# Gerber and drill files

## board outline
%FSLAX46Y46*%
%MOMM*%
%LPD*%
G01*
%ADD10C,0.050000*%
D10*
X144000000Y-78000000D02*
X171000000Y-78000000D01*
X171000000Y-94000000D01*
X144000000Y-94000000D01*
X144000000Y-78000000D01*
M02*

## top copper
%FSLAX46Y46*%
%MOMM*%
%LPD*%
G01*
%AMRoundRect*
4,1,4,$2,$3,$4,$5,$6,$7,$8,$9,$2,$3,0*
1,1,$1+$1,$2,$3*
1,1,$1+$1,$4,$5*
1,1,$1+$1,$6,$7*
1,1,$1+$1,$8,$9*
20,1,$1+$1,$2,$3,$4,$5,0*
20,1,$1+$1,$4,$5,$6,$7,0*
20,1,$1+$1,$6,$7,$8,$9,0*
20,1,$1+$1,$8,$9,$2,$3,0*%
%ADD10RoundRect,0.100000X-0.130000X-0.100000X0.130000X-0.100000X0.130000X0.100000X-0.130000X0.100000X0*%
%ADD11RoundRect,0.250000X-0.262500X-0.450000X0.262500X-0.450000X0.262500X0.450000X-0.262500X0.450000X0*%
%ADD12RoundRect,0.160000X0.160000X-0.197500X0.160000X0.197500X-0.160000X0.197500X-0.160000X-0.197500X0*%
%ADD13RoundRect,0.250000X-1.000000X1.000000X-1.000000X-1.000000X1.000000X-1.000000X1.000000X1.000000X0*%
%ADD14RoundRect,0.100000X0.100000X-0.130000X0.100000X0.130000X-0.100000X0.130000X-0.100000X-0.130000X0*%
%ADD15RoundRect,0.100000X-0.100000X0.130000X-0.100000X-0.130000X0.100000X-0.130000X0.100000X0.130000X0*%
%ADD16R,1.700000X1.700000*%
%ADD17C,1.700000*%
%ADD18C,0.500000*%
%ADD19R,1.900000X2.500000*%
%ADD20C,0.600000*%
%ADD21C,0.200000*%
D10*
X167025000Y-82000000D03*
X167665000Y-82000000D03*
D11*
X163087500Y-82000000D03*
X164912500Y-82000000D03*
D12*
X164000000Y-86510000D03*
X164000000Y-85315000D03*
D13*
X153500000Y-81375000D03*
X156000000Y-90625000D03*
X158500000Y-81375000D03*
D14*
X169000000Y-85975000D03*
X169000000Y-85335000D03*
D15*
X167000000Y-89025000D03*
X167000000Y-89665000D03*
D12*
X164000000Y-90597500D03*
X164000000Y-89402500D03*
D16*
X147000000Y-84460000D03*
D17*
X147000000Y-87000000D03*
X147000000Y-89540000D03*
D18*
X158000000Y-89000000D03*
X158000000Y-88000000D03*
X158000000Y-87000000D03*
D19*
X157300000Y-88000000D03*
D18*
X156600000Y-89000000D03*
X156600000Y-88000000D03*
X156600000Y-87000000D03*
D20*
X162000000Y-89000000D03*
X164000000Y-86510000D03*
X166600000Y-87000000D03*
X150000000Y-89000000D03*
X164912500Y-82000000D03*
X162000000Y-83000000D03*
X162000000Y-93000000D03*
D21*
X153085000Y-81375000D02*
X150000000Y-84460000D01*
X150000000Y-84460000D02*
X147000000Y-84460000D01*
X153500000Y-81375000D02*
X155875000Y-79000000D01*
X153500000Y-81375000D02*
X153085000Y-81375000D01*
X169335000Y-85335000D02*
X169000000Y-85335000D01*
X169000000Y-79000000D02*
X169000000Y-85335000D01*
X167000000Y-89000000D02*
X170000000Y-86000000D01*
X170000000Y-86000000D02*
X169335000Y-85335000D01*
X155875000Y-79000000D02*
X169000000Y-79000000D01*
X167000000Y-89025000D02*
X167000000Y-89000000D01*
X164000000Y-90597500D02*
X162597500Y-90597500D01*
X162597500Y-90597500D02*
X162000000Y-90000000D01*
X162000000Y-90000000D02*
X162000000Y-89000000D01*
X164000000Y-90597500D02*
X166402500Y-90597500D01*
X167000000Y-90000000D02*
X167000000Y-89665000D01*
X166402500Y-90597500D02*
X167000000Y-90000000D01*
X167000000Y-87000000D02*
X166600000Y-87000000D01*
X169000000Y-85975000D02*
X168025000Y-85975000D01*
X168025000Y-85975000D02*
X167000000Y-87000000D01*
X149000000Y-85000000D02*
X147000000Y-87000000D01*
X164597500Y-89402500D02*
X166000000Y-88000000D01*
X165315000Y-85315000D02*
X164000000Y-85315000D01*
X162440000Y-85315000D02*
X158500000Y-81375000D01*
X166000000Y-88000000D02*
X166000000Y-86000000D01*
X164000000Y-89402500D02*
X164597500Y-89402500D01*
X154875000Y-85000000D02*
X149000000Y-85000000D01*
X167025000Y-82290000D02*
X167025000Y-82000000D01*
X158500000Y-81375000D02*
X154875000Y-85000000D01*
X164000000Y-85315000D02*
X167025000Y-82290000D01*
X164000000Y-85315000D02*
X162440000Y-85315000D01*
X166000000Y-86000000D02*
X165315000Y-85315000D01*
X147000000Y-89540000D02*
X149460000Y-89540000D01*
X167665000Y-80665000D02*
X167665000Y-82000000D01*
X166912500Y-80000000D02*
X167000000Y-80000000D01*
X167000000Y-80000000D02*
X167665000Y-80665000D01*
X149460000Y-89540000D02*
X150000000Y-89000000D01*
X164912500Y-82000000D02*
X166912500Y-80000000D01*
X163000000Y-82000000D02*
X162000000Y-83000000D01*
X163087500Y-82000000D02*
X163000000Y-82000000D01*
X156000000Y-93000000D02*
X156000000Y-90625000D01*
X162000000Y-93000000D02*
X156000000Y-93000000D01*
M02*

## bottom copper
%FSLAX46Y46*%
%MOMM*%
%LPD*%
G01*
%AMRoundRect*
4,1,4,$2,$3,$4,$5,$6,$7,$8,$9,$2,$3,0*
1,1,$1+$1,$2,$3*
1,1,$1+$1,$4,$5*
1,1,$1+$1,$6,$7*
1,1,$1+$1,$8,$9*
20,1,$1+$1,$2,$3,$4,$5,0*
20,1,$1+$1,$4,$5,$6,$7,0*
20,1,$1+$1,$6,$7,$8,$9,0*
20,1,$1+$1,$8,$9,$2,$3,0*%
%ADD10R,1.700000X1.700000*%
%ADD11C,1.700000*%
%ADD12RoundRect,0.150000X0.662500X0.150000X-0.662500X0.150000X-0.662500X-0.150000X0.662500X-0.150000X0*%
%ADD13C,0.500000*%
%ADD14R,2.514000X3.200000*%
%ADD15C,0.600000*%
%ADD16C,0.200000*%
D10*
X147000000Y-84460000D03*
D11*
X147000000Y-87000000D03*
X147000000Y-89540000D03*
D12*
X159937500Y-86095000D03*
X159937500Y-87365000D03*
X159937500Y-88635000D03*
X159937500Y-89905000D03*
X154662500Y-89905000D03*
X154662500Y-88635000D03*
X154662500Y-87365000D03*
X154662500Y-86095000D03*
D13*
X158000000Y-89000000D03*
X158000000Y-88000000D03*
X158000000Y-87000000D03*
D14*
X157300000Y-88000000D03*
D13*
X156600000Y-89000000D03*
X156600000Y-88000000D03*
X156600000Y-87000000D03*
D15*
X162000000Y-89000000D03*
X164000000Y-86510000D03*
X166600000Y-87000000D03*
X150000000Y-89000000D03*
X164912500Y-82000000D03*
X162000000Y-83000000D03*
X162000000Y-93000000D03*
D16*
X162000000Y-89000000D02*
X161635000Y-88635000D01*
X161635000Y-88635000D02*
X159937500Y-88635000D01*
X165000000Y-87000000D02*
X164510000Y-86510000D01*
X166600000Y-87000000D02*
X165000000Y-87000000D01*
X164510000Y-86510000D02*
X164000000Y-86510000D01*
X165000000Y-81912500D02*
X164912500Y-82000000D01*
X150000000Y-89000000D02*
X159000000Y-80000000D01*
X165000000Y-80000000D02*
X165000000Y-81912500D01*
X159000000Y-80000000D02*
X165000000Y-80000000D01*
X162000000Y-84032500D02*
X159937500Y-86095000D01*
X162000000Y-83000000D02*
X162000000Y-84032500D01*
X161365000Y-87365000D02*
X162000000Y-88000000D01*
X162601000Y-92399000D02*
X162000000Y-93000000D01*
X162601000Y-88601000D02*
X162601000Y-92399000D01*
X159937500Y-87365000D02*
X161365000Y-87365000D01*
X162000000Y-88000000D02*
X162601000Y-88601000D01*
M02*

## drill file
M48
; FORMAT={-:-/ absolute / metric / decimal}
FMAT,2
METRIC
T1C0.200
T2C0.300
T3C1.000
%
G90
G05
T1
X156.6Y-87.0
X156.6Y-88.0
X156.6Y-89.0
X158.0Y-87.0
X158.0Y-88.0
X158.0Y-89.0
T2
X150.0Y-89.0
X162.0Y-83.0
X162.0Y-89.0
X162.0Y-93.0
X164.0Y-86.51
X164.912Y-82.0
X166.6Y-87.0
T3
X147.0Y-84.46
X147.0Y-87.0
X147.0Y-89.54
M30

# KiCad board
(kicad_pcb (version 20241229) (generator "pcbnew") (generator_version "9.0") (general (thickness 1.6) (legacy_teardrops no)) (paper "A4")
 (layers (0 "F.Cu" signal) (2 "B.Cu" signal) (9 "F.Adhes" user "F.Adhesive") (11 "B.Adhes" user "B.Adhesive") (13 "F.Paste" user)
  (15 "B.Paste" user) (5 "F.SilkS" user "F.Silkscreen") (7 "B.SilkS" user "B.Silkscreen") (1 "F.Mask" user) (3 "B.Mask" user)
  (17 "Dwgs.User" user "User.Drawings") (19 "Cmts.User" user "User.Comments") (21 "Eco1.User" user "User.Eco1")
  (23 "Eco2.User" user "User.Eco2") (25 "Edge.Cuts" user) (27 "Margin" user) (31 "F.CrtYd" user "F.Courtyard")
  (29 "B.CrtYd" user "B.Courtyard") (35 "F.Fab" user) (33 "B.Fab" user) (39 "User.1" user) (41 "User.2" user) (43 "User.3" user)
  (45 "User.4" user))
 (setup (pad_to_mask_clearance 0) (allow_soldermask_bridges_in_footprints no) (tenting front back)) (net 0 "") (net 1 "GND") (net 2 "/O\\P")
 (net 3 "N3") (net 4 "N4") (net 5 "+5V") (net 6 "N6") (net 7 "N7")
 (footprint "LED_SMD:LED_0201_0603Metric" (layer "F.Cu") (at 167.345 82)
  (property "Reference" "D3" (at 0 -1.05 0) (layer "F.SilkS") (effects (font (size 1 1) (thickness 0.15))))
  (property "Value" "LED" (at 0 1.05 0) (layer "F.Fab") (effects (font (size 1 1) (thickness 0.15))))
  (pad "" smd roundrect (at -0.345 0) (size 0.318 0.36) (layers "F.Paste") (roundrect_rratio 0.25))
  (pad "" smd roundrect (at 0.345 0) (size 0.318 0.36) (layers "F.Paste") (roundrect_rratio 0.25))
  (pad "1" smd roundrect (at -0.32 0) (size 0.46 0.4) (layers "F.Cu" "F.Mask") (roundrect_rratio 0.25) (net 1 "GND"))
  (pad "2" smd roundrect (at 0.32 0) (size 0.46 0.4) (layers "F.Cu" "F.Mask") (roundrect_rratio 0.25) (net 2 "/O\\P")))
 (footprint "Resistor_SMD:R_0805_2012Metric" (layer "F.Cu") (at 164 82)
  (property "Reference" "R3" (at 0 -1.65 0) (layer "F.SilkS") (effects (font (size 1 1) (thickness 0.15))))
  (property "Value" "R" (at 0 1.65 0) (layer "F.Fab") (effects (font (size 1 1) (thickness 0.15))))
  (pad "1" smd roundrect (at -0.9125 0) (size 1.025 1.4) (layers "F.Cu" "F.Mask" "F.Paste") (roundrect_rratio 0.243902) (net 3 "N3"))
  (pad "2" smd roundrect (at 0.9125 0) (size 1.025 1.4) (layers "F.Cu" "F.Mask" "F.Paste") (roundrect_rratio 0.243902) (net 2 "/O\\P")))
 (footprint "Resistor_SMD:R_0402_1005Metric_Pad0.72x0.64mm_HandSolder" (layer "F.Cu") (at 164 85.9125 90)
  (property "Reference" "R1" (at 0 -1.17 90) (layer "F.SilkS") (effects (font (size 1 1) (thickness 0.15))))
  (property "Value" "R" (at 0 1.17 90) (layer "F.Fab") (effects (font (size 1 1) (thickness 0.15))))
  (pad "1" smd roundrect (at -0.5975 0 90) (size 0.715 0.64) (layers "F.Cu" "F.Mask" "F.Paste") (roundrect_rratio 0.25) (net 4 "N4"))
  (pad "2" smd roundrect (at 0.5975 0 90) (size 0.715 0.64) (layers "F.Cu" "F.Mask" "F.Paste") (roundrect_rratio 0.25) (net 1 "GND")))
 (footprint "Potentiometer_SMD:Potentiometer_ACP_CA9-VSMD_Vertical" (layer "F.Cu") (at 156 86 -90)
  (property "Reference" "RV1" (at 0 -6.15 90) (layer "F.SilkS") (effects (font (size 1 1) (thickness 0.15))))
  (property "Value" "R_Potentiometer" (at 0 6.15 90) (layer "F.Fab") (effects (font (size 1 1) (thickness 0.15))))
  (pad "1" smd roundrect (at -4.625 2.5 270) (size 2.5 2.5) (layers "F.Cu" "F.Mask" "F.Paste") (roundrect_rratio 0.1) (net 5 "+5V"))
  (pad "2" smd roundrect (at 4.625 0 270) (size 2.5 2.5) (layers "F.Cu" "F.Mask" "F.Paste") (roundrect_rratio 0.1) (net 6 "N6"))
  (pad "3" smd roundrect (at -4.625 -2.5 270) (size 2.5 2.5) (layers "F.Cu" "F.Mask" "F.Paste") (roundrect_rratio 0.1) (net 1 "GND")))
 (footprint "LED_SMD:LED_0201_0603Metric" (layer "F.Cu") (at 169 85.655 90)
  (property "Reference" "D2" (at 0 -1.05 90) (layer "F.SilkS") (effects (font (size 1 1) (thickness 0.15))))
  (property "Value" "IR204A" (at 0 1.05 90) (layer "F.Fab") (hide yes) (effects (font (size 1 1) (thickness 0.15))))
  (pad "" smd roundrect (at -0.345 0 90) (size 0.318 0.36) (layers "F.Paste") (roundrect_rratio 0.25))
  (pad "" smd roundrect (at 0.345 0 90) (size 0.318 0.36) (layers "F.Paste") (roundrect_rratio 0.25))
  (pad "1" smd roundrect (at -0.32 0 90) (size 0.46 0.4) (layers "F.Cu" "F.Mask") (roundrect_rratio 0.25) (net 4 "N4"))
  (pad "2" smd roundrect (at 0.32 0 90) (size 0.46 0.4) (layers "F.Cu" "F.Mask") (roundrect_rratio 0.25) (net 5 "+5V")))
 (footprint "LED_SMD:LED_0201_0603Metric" (layer "F.Cu") (at 167 89.345 -90)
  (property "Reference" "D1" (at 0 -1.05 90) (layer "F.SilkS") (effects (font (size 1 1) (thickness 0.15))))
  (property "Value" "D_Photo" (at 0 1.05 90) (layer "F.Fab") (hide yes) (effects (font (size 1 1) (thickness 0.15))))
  (pad "" smd roundrect (at -0.345 0 270) (size 0.318 0.36) (layers "F.Paste") (roundrect_rratio 0.25))
  (pad "" smd roundrect (at 0.345 0 270) (size 0.318 0.36) (layers "F.Paste") (roundrect_rratio 0.25))
  (pad "1" smd roundrect (at -0.32 0 270) (size 0.46 0.4) (layers "F.Cu" "F.Mask") (roundrect_rratio 0.25) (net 5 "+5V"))
  (pad "2" smd roundrect (at 0.32 0 270) (size 0.46 0.4) (layers "F.Cu" "F.Mask") (roundrect_rratio 0.25) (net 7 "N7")))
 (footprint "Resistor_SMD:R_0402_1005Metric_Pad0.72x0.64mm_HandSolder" (layer "F.Cu") (at 164 90 90)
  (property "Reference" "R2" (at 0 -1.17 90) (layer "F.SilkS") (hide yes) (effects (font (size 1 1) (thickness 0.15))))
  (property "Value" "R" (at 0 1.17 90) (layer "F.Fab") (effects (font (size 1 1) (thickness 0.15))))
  (pad "1" smd roundrect (at -0.5975 0 90) (size 0.715 0.64) (layers "F.Cu" "F.Mask" "F.Paste") (roundrect_rratio 0.25) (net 7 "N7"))
  (pad "2" smd roundrect (at 0.5975 0 90) (size 0.715 0.64) (layers "F.Cu" "F.Mask" "F.Paste") (roundrect_rratio 0.25) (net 1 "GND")))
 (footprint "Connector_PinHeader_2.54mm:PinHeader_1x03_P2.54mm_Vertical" (layer "F.Cu") (at 147 84.46)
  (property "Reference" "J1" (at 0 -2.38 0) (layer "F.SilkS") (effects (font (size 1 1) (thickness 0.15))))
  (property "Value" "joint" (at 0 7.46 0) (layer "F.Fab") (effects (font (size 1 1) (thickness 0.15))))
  (pad "1" thru_hole rect (at 0 0) (size 1.7 1.7) (drill 1) (layers "*.Cu" "*.Mask") (remove_unused_layers no) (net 5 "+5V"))
  (pad "2" thru_hole circle (at 0 2.54) (size 1.7 1.7) (drill 1) (layers "*.Cu" "*.Mask") (remove_unused_layers no) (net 1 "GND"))
  (pad "3" thru_hole circle (at 0 5.08) (size 1.7 1.7) (drill 1) (layers "*.Cu" "*.Mask") (remove_unused_layers no) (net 2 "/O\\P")))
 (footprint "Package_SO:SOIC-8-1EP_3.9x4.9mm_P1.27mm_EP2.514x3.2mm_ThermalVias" (layer "B.Cu") (at 157.3 88 180)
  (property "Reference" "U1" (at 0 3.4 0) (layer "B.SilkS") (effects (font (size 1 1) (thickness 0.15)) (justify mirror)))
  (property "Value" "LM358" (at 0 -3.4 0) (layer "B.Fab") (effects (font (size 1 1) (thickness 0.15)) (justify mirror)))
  (pad "" smd roundrect (at -0.63 -0.8 180) (size 1.05 1.34) (layers "B.Paste") (roundrect_rratio 0.238095))
  (pad "" smd roundrect (at -0.63 0.8 180) (size 1.05 1.34) (layers "B.Paste") (roundrect_rratio 0.238095))
  (pad "" smd roundrect (at 0.63 -0.8 180) (size 1.05 1.34) (layers "B.Paste") (roundrect_rratio 0.238095))
  (pad "" smd roundrect (at 0.63 0.8 180) (size 1.05 1.34) (layers "B.Paste") (roundrect_rratio 0.238095))
  (pad "1" smd roundrect (at -2.6375 1.905 180) (size 1.625 0.6) (layers "B.Cu" "B.Mask" "B.Paste") (roundrect_rratio 0.25) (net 3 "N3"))
  (pad "2" smd roundrect (at -2.6375 0.635 180) (size 1.625 0.6) (layers "B.Cu" "B.Mask" "B.Paste") (roundrect_rratio 0.25) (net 6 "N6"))
  (pad "3" smd roundrect (at -2.6375 -0.635 180) (size 1.625 0.6) (layers "B.Cu" "B.Mask" "B.Paste") (roundrect_rratio 0.25) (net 7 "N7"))
  (pad "4" smd roundrect (at -2.6375 -1.905 180) (size 1.625 0.6) (layers "B.Cu" "B.Mask" "B.Paste") (roundrect_rratio 0.25))
  (pad "5" smd roundrect (at 2.6375 -1.905 180) (size 1.625 0.6) (layers "B.Cu" "B.Mask" "B.Paste") (roundrect_rratio 0.25))
  (pad "6" smd roundrect (at 2.6375 -0.635 180) (size 1.625 0.6) (layers "B.Cu" "B.Mask" "B.Paste") (roundrect_rratio 0.25))
  (pad "7" smd roundrect (at 2.6375 0.635 180) (size 1.625 0.6) (layers "B.Cu" "B.Mask" "B.Paste") (roundrect_rratio 0.25))
  (pad "8" smd roundrect (at 2.6375 1.905 180) (size 1.625 0.6) (layers "B.Cu" "B.Mask" "B.Paste") (roundrect_rratio 0.25))
  (pad "9" thru_hole circle (at -0.7 -1 180) (size 0.5 0.5) (drill 0.2) (layers "*.Cu") (remove_unused_layers no))
  (pad "9" thru_hole circle (at -0.7 0 180) (size 0.5 0.5) (drill 0.2) (layers "*.Cu") (remove_unused_layers no))
  (pad "9" thru_hole circle (at -0.7 1 180) (size 0.5 0.5) (drill 0.2) (layers "*.Cu") (remove_unused_layers no))
  (pad "9" smd rect (at 0 0 180) (size 1.9 2.5) (layers "F.Cu") (zone_connect 2))
  (pad "9" smd rect (at 0 0 180) (size 2.514 3.2) (layers "B.Cu" "B.Mask") (zone_connect 2))
  (pad "9" thru_hole circle (at 0.7 -1 180) (size 0.5 0.5) (drill 0.2) (layers "*.Cu") (remove_unused_layers no))
  (pad "9" thru_hole circle (at 0.7 0 180) (size 0.5 0.5) (drill 0.2) (layers "*.Cu") (remove_unused_layers no))
  (pad "9" thru_hole circle (at 0.7 1 180) (size 0.5 0.5) (drill 0.2) (layers "*.Cu") (remove_unused_layers no)))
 (gr_rect (start 144 78) (end 171 94) (stroke (width 0.05) (type default)) (fill no) (layer "Edge.Cuts"))
 (segment (start 153.085 81.375) (end 150 84.46) (width 0.2) (layer "F.Cu") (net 5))
 (segment (start 150 84.46) (end 147 84.46) (width 0.2) (layer "F.Cu") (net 5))
 (segment (start 153.5 81.375) (end 155.875 79) (width 0.2) (layer "F.Cu") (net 5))
 (segment (start 153.5 81.375) (end 153.085 81.375) (width 0.2) (layer "F.Cu") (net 5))
 (segment (start 169.335 85.335) (end 169 85.335) (width 0.2) (layer "F.Cu") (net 5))
 (segment (start 169 79) (end 169 85.335) (width 0.2) (layer "F.Cu") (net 5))
 (segment (start 167 89) (end 170 86) (width 0.2) (layer "F.Cu") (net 5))
 (segment (start 170 86) (end 169.335 85.335) (width 0.2) (layer "F.Cu") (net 5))
 (segment (start 155.875 79) (end 169 79) (width 0.2) (layer "F.Cu") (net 5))
 (segment (start 167 89.025) (end 167 89) (width 0.2) (layer "F.Cu") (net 5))
 (segment (start 164 90.5975) (end 162.5975 90.5975) (width 0.2) (layer "F.Cu") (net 7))
 (segment (start 162.5975 90.5975) (end 162 90) (width 0.2) (layer "F.Cu") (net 7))
 (segment (start 162 90) (end 162 89) (width 0.2) (layer "F.Cu") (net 7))
 (segment (start 164 90.5975) (end 166.4025 90.5975) (width 0.2) (layer "F.Cu") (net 7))
 (segment (start 167 90) (end 167 89.665) (width 0.2) (layer "F.Cu") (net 7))
 (segment (start 166.4025 90.5975) (end 167 90) (width 0.2) (layer "F.Cu") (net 7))
 (via (at 162 89) (size 0.6) (drill 0.3) (layers "F.Cu" "B.Cu") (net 7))
 (segment (start 162 89) (end 161.635 88.635) (width 0.2) (layer "B.Cu") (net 7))
 (segment (start 161.635 88.635) (end 159.9375 88.635) (width 0.2) (layer "B.Cu") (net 7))
 (segment (start 167 87) (end 166.6 87) (width 0.2) (layer "F.Cu") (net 4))
 (segment (start 169 85.975) (end 168.025 85.975) (width 0.2) (layer "F.Cu") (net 4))
 (segment (start 168.025 85.975) (end 167 87) (width 0.2) (layer "F.Cu") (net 4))
 (via (at 164 86.51) (size 0.6) (drill 0.3) (layers "F.Cu" "B.Cu") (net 4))
 (via (at 166.6 87) (size 0.6) (drill 0.3) (layers "F.Cu" "B.Cu") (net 4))
 (segment (start 165 87) (end 164.51 86.51) (width 0.2) (layer "B.Cu") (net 4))
 (segment (start 166.6 87) (end 165 87) (width 0.2) (layer "B.Cu") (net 4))
 (segment (start 164.51 86.51) (end 164 86.51) (width 0.2) (layer "B.Cu") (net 4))
 (segment (start 149 85) (end 147 87) (width 0.2) (layer "F.Cu") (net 1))
 (segment (start 164.5975 89.4025) (end 166 88) (width 0.2) (layer "F.Cu") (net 1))
 (segment (start 165.315 85.315) (end 164 85.315) (width 0.2) (layer "F.Cu") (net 1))
 (segment (start 162.44 85.315) (end 158.5 81.375) (width 0.2) (layer "F.Cu") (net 1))
 (segment (start 166 88) (end 166 86) (width 0.2) (layer "F.Cu") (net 1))
 (segment (start 164 89.4025) (end 164.5975 89.4025) (width 0.2) (layer "F.Cu") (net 1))
 (segment (start 154.875 85) (end 149 85) (width 0.2) (layer "F.Cu") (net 1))
 (segment (start 167.025 82.29) (end 167.025 82) (width 0.2) (layer "F.Cu") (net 1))
 (segment (start 158.5 81.375) (end 154.875 85) (width 0.2) (layer "F.Cu") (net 1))
 (segment (start 164 85.315) (end 167.025 82.29) (width 0.2) (layer "F.Cu") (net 1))
 (segment (start 164 85.315) (end 162.44 85.315) (width 0.2) (layer "F.Cu") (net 1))
 (segment (start 166 86) (end 165.315 85.315) (width 0.2) (layer "F.Cu") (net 1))
 (segment (start 147 89.54) (end 149.46 89.54) (width 0.2) (layer "F.Cu") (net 2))
 (segment (start 167.665 80.665) (end 167.665 82) (width 0.2) (layer "F.Cu") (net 2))
 (segment (start 166.9125 80) (end 167 80) (width 0.2) (layer "F.Cu") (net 2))
 (segment (start 167 80) (end 167.665 80.665) (width 0.2) (layer "F.Cu") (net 2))
 (segment (start 149.46 89.54) (end 150 89) (width 0.2) (layer "F.Cu") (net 2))
 (segment (start 164.9125 82) (end 166.9125 80) (width 0.2) (layer "F.Cu") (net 2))
 (via (at 150 89) (size 0.6) (drill 0.3) (layers "F.Cu" "B.Cu") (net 2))
 (via (at 164.9125 82) (size 0.6) (drill 0.3) (layers "F.Cu" "B.Cu") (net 2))
 (segment (start 165 81.9125) (end 164.9125 82) (width 0.2) (layer "B.Cu") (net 2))
 (segment (start 150 89) (end 159 80) (width 0.2) (layer "B.Cu") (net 2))
 (segment (start 165 80) (end 165 81.9125) (width 0.2) (layer "B.Cu") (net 2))
 (segment (start 159 80) (end 165 80) (width 0.2) (layer "B.Cu") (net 2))
 (segment (start 163 82) (end 162 83) (width 0.2) (layer "F.Cu") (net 3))
 (segment (start 163.0875 82) (end 163 82) (width 0.2) (layer "F.Cu") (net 3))
 (via (at 162 83) (size 0.6) (drill 0.3) (layers "F.Cu" "B.Cu") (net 3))
 (segment (start 162 84.0325) (end 159.9375 86.095) (width 0.2) (layer "B.Cu") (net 3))
 (segment (start 162 83) (end 162 84.0325) (width 0.2) (layer "B.Cu") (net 3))
 (segment (start 156 93) (end 156 90.625) (width 0.2) (layer "F.Cu") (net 6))
 (segment (start 162 93) (end 156 93) (width 0.2) (layer "F.Cu") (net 6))
 (via (at 162 93) (size 0.6) (drill 0.3) (layers "F.Cu" "B.Cu") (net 6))
 (segment (start 161.365 87.365) (end 162 88) (width 0.2) (layer "B.Cu") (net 6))
 (segment (start 162.601 92.399) (end 162 93) (width 0.2) (layer "B.Cu") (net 6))
 (segment (start 162.601 88.601) (end 162.601 92.399) (width 0.2) (layer "B.Cu") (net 6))
 (segment (start 159.9375 87.365) (end 161.365 87.365) (width 0.2) (layer "B.Cu") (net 6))
 (segment (start 162 88) (end 162.601 88.601) (width 0.2) (layer "B.Cu") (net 6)))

